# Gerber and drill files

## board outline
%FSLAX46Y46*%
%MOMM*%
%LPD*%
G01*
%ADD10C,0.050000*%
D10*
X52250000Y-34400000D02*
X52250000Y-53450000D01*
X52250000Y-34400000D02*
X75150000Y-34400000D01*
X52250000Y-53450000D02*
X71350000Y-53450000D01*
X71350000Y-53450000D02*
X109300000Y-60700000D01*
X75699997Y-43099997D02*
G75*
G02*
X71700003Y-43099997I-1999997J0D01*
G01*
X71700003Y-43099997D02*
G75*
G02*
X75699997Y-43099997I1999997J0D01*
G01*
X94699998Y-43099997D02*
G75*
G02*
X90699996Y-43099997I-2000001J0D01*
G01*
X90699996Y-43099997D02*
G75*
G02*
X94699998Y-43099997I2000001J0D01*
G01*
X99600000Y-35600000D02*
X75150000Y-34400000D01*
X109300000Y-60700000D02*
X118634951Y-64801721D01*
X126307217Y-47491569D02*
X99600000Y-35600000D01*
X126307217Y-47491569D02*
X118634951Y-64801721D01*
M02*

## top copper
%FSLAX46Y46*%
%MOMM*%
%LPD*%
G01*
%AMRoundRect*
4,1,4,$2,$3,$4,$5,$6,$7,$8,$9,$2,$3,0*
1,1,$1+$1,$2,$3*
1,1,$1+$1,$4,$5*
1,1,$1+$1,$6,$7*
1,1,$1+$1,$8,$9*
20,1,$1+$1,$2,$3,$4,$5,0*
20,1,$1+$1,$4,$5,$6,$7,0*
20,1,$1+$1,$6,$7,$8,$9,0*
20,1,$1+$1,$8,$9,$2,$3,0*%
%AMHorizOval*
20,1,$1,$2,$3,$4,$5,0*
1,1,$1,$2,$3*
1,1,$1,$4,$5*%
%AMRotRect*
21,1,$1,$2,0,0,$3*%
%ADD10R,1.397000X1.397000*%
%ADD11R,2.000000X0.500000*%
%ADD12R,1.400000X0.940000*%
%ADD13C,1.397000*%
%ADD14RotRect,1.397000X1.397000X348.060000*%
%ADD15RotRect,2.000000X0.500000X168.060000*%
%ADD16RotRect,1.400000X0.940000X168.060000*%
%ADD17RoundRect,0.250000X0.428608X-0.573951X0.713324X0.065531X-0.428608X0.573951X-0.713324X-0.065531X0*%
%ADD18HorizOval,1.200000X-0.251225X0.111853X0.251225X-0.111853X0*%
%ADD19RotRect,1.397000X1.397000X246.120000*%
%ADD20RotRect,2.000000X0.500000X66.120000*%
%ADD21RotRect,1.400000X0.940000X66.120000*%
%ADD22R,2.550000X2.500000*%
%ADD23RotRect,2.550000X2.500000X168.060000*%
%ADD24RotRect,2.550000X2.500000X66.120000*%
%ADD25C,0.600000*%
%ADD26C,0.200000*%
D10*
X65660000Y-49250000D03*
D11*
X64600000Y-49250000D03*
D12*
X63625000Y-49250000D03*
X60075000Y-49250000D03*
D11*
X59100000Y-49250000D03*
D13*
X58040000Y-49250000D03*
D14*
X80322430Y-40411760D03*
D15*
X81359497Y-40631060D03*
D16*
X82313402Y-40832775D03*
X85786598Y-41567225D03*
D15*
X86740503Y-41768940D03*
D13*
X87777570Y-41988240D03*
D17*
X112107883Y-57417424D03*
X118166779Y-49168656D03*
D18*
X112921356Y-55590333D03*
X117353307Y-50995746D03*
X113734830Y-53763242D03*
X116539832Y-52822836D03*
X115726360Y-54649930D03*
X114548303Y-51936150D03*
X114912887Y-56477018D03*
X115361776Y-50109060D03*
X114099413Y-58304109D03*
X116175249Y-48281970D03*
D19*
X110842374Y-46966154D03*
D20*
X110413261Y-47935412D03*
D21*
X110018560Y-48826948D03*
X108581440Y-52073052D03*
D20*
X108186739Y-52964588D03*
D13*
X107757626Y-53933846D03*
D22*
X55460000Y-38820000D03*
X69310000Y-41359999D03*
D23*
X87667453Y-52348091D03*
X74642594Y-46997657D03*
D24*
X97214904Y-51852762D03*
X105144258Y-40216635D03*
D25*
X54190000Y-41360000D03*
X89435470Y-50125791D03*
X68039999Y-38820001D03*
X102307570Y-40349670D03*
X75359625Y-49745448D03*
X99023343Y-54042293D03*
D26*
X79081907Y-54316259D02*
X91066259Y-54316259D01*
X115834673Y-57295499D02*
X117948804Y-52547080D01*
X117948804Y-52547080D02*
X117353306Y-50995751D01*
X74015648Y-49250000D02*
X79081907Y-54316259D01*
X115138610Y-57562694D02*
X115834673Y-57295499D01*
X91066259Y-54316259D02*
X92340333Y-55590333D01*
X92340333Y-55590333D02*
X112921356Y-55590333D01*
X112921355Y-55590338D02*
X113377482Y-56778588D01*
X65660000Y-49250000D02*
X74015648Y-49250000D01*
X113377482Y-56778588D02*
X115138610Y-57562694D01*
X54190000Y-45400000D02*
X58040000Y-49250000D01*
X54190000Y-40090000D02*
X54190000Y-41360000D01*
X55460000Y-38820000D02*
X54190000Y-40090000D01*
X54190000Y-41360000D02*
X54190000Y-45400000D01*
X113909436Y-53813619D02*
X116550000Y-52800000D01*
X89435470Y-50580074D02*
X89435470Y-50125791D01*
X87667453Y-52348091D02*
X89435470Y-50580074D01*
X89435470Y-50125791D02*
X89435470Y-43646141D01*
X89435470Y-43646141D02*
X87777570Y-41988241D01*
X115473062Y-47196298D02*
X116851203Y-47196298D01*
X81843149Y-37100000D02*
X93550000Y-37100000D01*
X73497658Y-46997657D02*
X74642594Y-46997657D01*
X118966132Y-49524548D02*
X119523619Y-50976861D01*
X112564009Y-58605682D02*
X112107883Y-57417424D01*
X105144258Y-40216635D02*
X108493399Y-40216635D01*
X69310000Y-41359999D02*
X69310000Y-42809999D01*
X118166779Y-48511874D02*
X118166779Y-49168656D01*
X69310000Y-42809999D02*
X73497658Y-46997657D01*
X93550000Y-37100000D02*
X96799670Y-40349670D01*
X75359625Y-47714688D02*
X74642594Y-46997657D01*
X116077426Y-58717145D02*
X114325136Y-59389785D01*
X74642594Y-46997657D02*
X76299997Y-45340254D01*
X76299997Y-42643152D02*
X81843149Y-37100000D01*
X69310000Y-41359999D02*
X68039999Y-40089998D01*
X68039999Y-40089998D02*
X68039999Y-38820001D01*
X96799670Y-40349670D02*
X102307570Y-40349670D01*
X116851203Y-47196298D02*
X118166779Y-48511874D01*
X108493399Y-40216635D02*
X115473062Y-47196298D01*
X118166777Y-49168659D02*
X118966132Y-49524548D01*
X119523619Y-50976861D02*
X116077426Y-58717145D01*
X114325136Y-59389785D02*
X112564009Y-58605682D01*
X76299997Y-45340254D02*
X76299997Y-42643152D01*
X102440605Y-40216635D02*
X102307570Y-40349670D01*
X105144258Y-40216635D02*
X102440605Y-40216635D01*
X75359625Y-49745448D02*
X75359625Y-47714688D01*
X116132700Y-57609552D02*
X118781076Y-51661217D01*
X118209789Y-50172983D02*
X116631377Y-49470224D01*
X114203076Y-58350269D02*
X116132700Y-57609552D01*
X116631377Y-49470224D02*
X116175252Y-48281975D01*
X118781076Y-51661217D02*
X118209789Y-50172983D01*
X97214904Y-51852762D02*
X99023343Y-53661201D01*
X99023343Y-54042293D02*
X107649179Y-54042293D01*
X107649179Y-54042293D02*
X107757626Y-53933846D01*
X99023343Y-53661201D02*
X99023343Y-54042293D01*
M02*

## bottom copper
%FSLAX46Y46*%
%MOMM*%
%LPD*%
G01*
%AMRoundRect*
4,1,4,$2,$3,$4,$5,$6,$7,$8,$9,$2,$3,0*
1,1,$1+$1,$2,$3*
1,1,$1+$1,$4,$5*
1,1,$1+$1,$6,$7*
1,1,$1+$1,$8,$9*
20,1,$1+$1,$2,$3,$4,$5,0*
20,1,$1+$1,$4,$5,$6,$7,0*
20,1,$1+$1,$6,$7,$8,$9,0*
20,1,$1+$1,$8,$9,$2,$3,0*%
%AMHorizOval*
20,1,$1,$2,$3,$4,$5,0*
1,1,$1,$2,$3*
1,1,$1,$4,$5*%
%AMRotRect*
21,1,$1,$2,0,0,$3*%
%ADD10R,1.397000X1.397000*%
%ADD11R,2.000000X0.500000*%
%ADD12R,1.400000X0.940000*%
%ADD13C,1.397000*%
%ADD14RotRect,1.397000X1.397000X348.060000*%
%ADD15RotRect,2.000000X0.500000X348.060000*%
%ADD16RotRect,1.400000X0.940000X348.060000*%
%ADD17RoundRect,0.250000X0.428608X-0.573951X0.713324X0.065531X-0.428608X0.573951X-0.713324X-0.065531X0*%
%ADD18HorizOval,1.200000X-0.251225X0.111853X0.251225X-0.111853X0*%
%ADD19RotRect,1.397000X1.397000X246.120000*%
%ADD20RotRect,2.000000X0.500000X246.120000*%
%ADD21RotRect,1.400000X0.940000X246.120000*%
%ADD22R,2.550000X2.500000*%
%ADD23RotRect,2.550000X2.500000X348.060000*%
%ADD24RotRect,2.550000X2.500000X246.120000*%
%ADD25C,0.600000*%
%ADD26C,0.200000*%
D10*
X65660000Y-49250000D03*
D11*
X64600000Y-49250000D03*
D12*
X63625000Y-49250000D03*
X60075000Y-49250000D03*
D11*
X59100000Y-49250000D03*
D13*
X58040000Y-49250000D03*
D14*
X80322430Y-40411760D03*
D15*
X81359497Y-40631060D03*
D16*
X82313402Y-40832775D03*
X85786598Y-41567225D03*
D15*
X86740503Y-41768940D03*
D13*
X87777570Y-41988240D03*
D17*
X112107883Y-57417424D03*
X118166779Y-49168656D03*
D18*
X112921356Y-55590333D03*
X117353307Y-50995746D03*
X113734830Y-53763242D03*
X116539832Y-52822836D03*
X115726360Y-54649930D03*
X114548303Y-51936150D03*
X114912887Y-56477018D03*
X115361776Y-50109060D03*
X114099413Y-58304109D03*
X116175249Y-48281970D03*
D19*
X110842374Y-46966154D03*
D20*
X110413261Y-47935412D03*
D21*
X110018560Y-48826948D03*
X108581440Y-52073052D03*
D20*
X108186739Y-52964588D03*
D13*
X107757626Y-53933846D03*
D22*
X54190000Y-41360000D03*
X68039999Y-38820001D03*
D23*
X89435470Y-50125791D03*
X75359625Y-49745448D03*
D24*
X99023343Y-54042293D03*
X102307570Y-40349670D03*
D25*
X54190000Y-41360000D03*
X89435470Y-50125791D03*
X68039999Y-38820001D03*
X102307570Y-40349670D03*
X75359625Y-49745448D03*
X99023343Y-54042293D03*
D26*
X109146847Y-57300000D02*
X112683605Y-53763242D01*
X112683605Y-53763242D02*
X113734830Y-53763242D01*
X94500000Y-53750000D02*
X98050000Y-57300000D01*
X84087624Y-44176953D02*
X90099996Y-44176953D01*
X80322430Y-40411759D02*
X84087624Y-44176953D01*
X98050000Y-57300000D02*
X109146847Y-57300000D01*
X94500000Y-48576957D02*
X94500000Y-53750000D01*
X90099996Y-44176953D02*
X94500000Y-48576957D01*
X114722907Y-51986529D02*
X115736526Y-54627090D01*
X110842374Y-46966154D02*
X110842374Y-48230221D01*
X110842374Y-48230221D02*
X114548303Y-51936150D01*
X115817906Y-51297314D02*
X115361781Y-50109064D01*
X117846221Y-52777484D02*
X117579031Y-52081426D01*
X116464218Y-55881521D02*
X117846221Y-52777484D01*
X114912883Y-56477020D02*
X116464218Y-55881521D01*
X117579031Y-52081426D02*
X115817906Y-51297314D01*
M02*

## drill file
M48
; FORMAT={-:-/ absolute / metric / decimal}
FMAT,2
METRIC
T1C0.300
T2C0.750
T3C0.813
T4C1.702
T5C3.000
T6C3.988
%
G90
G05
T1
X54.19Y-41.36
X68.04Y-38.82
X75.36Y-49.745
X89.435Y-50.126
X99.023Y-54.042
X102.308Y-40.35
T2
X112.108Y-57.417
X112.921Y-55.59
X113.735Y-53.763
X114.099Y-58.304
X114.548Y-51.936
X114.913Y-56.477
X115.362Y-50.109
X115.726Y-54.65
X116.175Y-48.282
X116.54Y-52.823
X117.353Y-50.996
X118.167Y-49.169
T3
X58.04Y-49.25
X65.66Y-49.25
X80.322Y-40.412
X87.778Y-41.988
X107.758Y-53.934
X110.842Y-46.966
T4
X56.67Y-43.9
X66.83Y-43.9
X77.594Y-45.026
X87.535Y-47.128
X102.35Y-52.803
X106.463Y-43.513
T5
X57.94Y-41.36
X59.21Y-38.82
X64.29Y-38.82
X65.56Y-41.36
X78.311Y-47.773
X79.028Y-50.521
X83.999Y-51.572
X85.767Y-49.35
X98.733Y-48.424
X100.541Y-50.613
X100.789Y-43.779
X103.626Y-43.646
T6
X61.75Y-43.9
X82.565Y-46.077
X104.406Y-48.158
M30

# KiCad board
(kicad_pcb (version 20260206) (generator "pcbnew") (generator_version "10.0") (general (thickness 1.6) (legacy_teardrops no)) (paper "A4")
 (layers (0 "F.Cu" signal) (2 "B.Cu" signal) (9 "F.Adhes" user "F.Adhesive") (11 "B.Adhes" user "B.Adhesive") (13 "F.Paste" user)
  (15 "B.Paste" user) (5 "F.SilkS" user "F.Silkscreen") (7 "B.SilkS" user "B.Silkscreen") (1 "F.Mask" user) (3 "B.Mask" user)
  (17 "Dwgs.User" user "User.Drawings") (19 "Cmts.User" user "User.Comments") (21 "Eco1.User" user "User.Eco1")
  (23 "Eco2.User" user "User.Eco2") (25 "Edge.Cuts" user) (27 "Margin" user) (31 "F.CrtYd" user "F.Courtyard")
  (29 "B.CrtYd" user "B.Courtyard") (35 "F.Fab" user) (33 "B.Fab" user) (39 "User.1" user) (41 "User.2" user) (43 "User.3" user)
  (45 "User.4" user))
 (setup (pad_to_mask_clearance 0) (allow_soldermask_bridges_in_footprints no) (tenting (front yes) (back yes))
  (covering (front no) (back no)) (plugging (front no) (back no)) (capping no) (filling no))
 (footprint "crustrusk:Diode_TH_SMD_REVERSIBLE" (layer "F.Cu") (at 61.85 49.25 180)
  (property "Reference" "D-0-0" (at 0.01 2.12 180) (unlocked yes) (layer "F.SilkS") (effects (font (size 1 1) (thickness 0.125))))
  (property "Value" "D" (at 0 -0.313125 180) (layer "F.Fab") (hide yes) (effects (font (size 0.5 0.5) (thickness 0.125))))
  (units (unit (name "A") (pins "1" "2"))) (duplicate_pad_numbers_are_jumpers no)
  (pad "1" thru_hole rect (at -3.81 0 180) (size 1.397 1.397) (drill 0.8128) (layers "*.Cu" "*.Mask") (remove_unused_layers no)
   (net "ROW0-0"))
  (pad "1" smd rect (at -2.75 0) (size 2 0.5) (layers "F.Cu") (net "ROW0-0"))
  (pad "1" smd rect (at -2.75 0 180) (size 2 0.5) (layers "B.Cu") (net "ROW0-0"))
  (pad "1" smd rect (at -1.775 0) (size 1.4 0.94) (layers "F.Cu" "F.Mask" "F.Paste") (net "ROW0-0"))
  (pad "1" smd rect (at -1.775 0 180) (size 1.4 0.94) (layers "B.Cu" "B.Mask" "B.Paste") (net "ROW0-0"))
  (pad "2" smd rect (at 1.775 0) (size 1.4 0.94) (layers "F.Cu" "F.Mask" "F.Paste") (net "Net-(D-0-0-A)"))
  (pad "2" smd rect (at 1.775 0 180) (size 1.4 0.94) (layers "B.Cu" "B.Mask" "B.Paste") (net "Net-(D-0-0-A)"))
  (pad "2" smd rect (at 2.75 0) (size 2 0.5) (layers "F.Cu") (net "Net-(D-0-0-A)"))
  (pad "2" smd rect (at 2.75 0 180) (size 2 0.5) (layers "B.Cu") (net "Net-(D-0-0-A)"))
  (pad "2" thru_hole circle (at 3.81 0 180) (size 1.397 1.397) (drill 0.8128) (layers "*.Cu" "*.Mask") (remove_unused_layers no)
   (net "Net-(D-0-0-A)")))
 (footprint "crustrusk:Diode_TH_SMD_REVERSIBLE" (layer "F.Cu") (at 84.05 41.2 -11.94)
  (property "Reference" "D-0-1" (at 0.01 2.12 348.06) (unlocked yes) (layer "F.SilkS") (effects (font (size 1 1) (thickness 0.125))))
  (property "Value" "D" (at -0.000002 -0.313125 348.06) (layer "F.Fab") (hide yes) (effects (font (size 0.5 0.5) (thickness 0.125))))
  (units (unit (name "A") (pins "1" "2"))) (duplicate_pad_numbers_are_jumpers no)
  (pad "1" thru_hole rect (at -3.81 0 348.06) (size 1.397 1.397) (drill 0.8128) (layers "*.Cu" "*.Mask") (remove_unused_layers no)
   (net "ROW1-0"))
  (pad "1" smd rect (at -2.75 0 168.06) (size 2 0.5) (layers "F.Cu") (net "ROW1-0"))
  (pad "1" smd rect (at -2.75 0 348.06) (size 2 0.5) (layers "B.Cu") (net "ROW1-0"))
  (pad "1" smd rect (at -1.775001 0 168.06) (size 1.4 0.94) (layers "F.Cu" "F.Mask" "F.Paste") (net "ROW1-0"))
  (pad "1" smd rect (at -1.775001 0 348.06) (size 1.4 0.94) (layers "B.Cu" "B.Mask" "B.Paste") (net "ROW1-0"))
  (pad "2" smd rect (at 1.775001 0 168.06) (size 1.4 0.94) (layers "F.Cu" "F.Mask" "F.Paste") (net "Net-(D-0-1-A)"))
  (pad "2" smd rect (at 1.775001 0 348.06) (size 1.4 0.94) (layers "B.Cu" "B.Mask" "B.Paste") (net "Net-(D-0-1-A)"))
  (pad "2" smd rect (at 2.75 0 168.06) (size 2 0.5) (layers "F.Cu") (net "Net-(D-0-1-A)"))
  (pad "2" smd rect (at 2.75 0 348.06) (size 2 0.5) (layers "B.Cu") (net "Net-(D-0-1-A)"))
  (pad "2" thru_hole circle (at 3.81 0 348.06) (size 1.397 1.397) (drill 0.8128) (layers "*.Cu" "*.Mask") (remove_unused_layers no)
   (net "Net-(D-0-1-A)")))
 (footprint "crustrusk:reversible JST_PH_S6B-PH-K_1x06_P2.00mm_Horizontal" (layer "F.Cu") (at 112.107883 57.417424 66)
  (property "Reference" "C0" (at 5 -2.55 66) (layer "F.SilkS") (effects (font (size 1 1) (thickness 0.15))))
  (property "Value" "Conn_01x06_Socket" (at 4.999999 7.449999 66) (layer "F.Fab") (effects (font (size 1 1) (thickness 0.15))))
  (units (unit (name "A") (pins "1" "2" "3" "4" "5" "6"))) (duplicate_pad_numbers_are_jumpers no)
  (pad "1" thru_hole roundrect (at 0 0 66) (size 1.2 1.75) (drill 0.75) (layers "*.Cu" "*.Mask") (remove_unused_layers no)
   (roundrect_rratio 0.208333) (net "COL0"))
  (pad "1" thru_hole roundrect (at 10 2.180001 66) (size 1.2 1.75) (drill 0.75) (layers "*.Cu" "*.Mask") (remove_unused_layers no)
   (roundrect_rratio 0.208333) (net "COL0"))
  (pad "2" thru_hole oval (at 2 0 66) (size 1.2 1.75) (drill 0.75) (layers "*.Cu" "*.Mask") (remove_unused_layers no) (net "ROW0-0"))
  (pad "2" thru_hole oval (at 8.000001 2.180002 66) (size 1.2 1.75) (drill 0.75) (layers "*.Cu" "*.Mask") (remove_unused_layers no)
   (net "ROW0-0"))
  (pad "3" thru_hole oval (at 4 0 66) (size 1.2 1.75) (drill 0.75) (layers "*.Cu" "*.Mask") (remove_unused_layers no) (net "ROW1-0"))
  (pad "3" thru_hole oval (at 6.000001 2.18 66) (size 1.2 1.75) (drill 0.75) (layers "*.Cu" "*.Mask") (remove_unused_layers no)
   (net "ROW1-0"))
  (pad "4" thru_hole oval (at 3.999999 2.180002 66) (size 1.2 1.75) (drill 0.75) (layers "*.Cu" "*.Mask") (remove_unused_layers no)
   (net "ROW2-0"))
  (pad "4" thru_hole oval (at 6.000001 0 66) (size 1.2 1.75) (drill 0.75) (layers "*.Cu" "*.Mask") (remove_unused_layers no) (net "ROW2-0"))
  (pad "5" thru_hole oval (at 2.000002 2.180001 66) (size 1.2 1.75) (drill 0.75) (layers "*.Cu" "*.Mask") (remove_unused_layers no)
   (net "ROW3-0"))
  (pad "5" thru_hole oval (at 8 0 66) (size 1.2 1.75) (drill 0.75) (layers "*.Cu" "*.Mask") (remove_unused_layers no) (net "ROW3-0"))
  (pad "6" thru_hole oval (at 0.000001 2.18 66) (size 1.2 1.75) (drill 0.75) (layers "*.Cu" "*.Mask") (remove_unused_layers no)
   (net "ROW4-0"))
  (pad "6" thru_hole oval (at 9.999999 0 66) (size 1.2 1.75) (drill 0.75) (layers "*.Cu" "*.Mask") (remove_unused_layers no) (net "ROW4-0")))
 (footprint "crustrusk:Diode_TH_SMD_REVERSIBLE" (layer "F.Cu") (at 109.3 50.45 -113.88)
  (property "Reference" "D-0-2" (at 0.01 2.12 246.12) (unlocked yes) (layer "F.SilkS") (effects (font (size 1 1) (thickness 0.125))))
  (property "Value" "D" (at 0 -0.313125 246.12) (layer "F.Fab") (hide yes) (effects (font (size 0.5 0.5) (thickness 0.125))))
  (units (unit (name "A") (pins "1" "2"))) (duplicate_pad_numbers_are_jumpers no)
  (pad "1" thru_hole rect (at -3.81 -0.000001 246.12) (size 1.397 1.397) (drill 0.8128) (layers "*.Cu" "*.Mask") (remove_unused_layers no)
   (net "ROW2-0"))
  (pad "1" smd rect (at -2.75 0.000001 66.12) (size 2 0.5) (layers "F.Cu") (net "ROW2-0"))
  (pad "1" smd rect (at -2.75 0.000001 246.12) (size 2 0.5) (layers "B.Cu") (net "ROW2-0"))
  (pad "1" smd rect (at -1.775 0 66.12) (size 1.4 0.94) (layers "F.Cu" "F.Mask" "F.Paste") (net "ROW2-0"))
  (pad "1" smd rect (at -1.775 0 246.12) (size 1.4 0.94) (layers "B.Cu" "B.Mask" "B.Paste") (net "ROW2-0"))
  (pad "2" smd rect (at 1.775 0 66.12) (size 1.4 0.94) (layers "F.Cu" "F.Mask" "F.Paste") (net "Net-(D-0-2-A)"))
  (pad "2" smd rect (at 1.775 0 246.12) (size 1.4 0.94) (layers "B.Cu" "B.Mask" "B.Paste") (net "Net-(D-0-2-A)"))
  (pad "2" smd rect (at 2.75 -0.000001 66.12) (size 2 0.5) (layers "F.Cu") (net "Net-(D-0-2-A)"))
  (pad "2" smd rect (at 2.75 -0.000001 246.12) (size 2 0.5) (layers "B.Cu") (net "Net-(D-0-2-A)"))
  (pad "2" thru_hole circle (at 3.81 0.000001 246.12) (size 1.397 1.397) (drill 0.8128) (layers "*.Cu" "*.Mask") (remove_unused_layers no)
   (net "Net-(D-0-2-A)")))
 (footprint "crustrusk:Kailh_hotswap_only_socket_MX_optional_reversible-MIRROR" (layer "B.Cu") (at 61.75 43.9 180)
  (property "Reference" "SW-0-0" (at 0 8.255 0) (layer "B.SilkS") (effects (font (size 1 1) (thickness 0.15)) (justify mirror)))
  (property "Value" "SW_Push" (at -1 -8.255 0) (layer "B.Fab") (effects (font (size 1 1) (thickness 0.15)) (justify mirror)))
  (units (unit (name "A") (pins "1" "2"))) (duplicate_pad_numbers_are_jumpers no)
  (pad "" np_thru_hole circle (at -5.08 0 180) (size 1.7018 1.7018) (drill 1.7018) (layers "*.Cu" "*.Mask"))
  (pad "" np_thru_hole circle (at -3.81 2.54) (size 3 3) (drill 3) (layers "*.Cu" "*.Mask"))
  (pad "" np_thru_hole circle (at -2.54 5.079998 180) (size 3 3) (drill 3) (layers "*.Cu" "*.Mask"))
  (pad "" np_thru_hole circle (at 0 0 180) (size 3.9878 3.9878) (drill 3.9878) (layers "*.Cu" "*.Mask"))
  (pad "" np_thru_hole circle (at 2.540002 5.080001) (size 3 3) (drill 3) (layers "*.Cu" "*.Mask"))
  (pad "" np_thru_hole circle (at 3.81 2.54 180) (size 3 3) (drill 3) (layers "*.Cu" "*.Mask"))
  (pad "" np_thru_hole circle (at 5.08 0 180) (size 1.7018 1.7018) (drill 1.7018) (layers "*.Cu" "*.Mask"))
  (pad "1" smd rect (at 6.29 5.08) (size 2.55 2.5) (layers "F.Cu" "F.Mask" "F.Paste") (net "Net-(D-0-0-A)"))
  (pad "1" smd rect (at 7.56 2.54 180) (size 2.55 2.5) (layers "B.Cu" "B.Mask" "B.Paste") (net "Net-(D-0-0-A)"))
  (pad "2" smd rect (at -7.56 2.540001) (size 2.55 2.5) (layers "F.Cu" "F.Mask" "F.Paste") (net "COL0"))
  (pad "2" smd rect (at -6.289999 5.079999 180) (size 2.55 2.5) (layers "B.Cu" "B.Mask" "B.Paste") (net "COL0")))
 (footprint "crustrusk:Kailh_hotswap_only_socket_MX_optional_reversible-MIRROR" (layer "B.Cu") (at 82.564526 46.076677 -11.94)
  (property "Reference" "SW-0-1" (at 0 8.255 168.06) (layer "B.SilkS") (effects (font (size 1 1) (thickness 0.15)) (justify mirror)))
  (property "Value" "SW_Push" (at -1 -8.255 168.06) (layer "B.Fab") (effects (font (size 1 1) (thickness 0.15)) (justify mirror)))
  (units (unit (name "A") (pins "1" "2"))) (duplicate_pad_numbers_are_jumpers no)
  (pad "" np_thru_hole circle (at -5.079999 0 348.06) (size 1.7018 1.7018) (drill 1.7018) (layers "*.Cu" "*.Mask"))
  (pad "" np_thru_hole circle (at -3.81 2.54 168.06) (size 3 3) (drill 3) (layers "*.Cu" "*.Mask"))
  (pad "" np_thru_hole circle (at -2.54 5.079997 348.06) (size 3 3) (drill 3) (layers "*.Cu" "*.Mask"))
  (pad "" np_thru_hole circle (at 0 0 348.06) (size 3.9878 3.9878) (drill 3.9878) (layers "*.Cu" "*.Mask"))
  (pad "" np_thru_hole circle (at 2.540002 5.080001 168.06) (size 3 3) (drill 3) (layers "*.Cu" "*.Mask"))
  (pad "" np_thru_hole circle (at 3.81 2.54 348.06) (size 3 3) (drill 3) (layers "*.Cu" "*.Mask"))
  (pad "" np_thru_hole circle (at 5.079999 0 348.06) (size 1.7018 1.7018) (drill 1.7018) (layers "*.Cu" "*.Mask"))
  (pad "1" smd rect (at 6.29 5.08 168.06) (size 2.55 2.5) (layers "F.Cu" "F.Mask" "F.Paste") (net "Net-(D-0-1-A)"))
  (pad "1" smd rect (at 7.56 2.54 348.06) (size 2.55 2.5) (layers "B.Cu" "B.Mask" "B.Paste") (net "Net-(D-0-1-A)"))
  (pad "2" smd rect (at -7.56 2.540001 168.06) (size 2.55 2.5) (layers "F.Cu" "F.Mask" "F.Paste") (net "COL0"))
  (pad "2" smd rect (at -6.289999 5.079999 348.06) (size 2.55 2.5) (layers "B.Cu" "B.Mask" "B.Paste") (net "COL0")))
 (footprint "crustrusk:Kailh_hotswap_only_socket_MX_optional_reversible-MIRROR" (layer "B.Cu") (at 104.406365 48.157713 -113.88)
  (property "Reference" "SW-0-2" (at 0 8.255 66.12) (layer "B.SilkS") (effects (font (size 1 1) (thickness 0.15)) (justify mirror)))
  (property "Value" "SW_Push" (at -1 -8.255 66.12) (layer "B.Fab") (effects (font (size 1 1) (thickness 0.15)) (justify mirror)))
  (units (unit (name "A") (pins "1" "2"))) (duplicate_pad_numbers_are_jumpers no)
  (pad "" np_thru_hole circle (at -5.08 0 246.12) (size 1.7018 1.7018) (drill 1.7018) (layers "*.Cu" "*.Mask"))
  (pad "" np_thru_hole circle (at -3.81 2.54 66.12) (size 3 3) (drill 3) (layers "*.Cu" "*.Mask"))
  (pad "" np_thru_hole circle (at -2.54 5.079998 246.12) (size 3 3) (drill 3) (layers "*.Cu" "*.Mask"))
  (pad "" np_thru_hole circle (at 0 0 246.12) (size 3.9878 3.9878) (drill 3.9878) (layers "*.Cu" "*.Mask"))
  (pad "" np_thru_hole circle (at 2.540002 5.080001 66.12) (size 3 3) (drill 3) (layers "*.Cu" "*.Mask"))
  (pad "" np_thru_hole circle (at 3.81 2.54 246.12) (size 3 3) (drill 3) (layers "*.Cu" "*.Mask"))
  (pad "" np_thru_hole circle (at 5.08 0 246.12) (size 1.7018 1.7018) (drill 1.7018) (layers "*.Cu" "*.Mask"))
  (pad "1" smd rect (at 6.29 5.08 66.12) (size 2.55 2.5) (layers "F.Cu" "F.Mask" "F.Paste") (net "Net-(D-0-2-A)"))
  (pad "1" smd rect (at 7.56 2.54 246.12) (size 2.55 2.5) (layers "B.Cu" "B.Mask" "B.Paste") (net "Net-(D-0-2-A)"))
  (pad "2" smd rect (at -7.56 2.540001 66.12) (size 2.55 2.5) (layers "F.Cu" "F.Mask" "F.Paste") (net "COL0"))
  (pad "2" smd rect (at -6.289999 5.079999 246.12) (size 2.55 2.5) (layers "B.Cu" "B.Mask" "B.Paste") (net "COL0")))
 (gr_line (start 52.25 34.4) (end 52.25 53.45) (stroke (width 0.05) (type default)) (layer "Edge.Cuts"))
 (gr_line (start 52.25 34.4) (end 75.15 34.4) (stroke (width 0.05) (type default)) (layer "Edge.Cuts"))
 (gr_line (start 52.25 53.45) (end 71.35 53.45) (stroke (width 0.05) (type default)) (layer "Edge.Cuts"))
 (gr_line (start 71.35 53.45) (end 109.3 60.7) (stroke (width 0.05) (type default)) (layer "Edge.Cuts"))
 (gr_circle (center 73.7 43.099997) (end 75.699997 43.099997) (stroke (width 0.05) (type default)) (fill no) (layer "Edge.Cuts"))
 (gr_circle (center 92.699997 43.099997) (end 94.699998 43.099997) (stroke (width 0.05) (type default)) (fill no) (layer "Edge.Cuts"))
 (gr_line (start 99.6 35.6) (end 75.15 34.4) (stroke (width 0.05) (type default)) (layer "Edge.Cuts"))
 (gr_line (start 109.3 60.7) (end 118.634951 64.801721) (stroke (width 0.05) (type default)) (layer "Edge.Cuts"))
 (gr_line (start 126.307217 47.491569) (end 99.6 35.6) (stroke (width 0.05) (type default)) (layer "Edge.Cuts"))
 (gr_line (start 126.307217 47.491569) (end 118.634951 64.801721) (stroke (width 0.05) (type default)) (layer "Edge.Cuts"))
 (segment (start 79.081907 54.316259) (end 91.066259 54.316259) (width 0.2) (layer "F.Cu") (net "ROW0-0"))
 (segment (start 115.834673 57.295499) (end 117.948804 52.54708) (width 0.2) (layer "F.Cu") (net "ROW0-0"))
 (segment (start 117.948804 52.54708) (end 117.353306 50.995751) (width 0.2) (layer "F.Cu") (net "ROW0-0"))
 (segment (start 74.015648 49.25) (end 79.081907 54.316259) (width 0.2) (layer "F.Cu") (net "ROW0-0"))
 (segment (start 115.13861 57.562694) (end 115.834673 57.295499) (width 0.2) (layer "F.Cu") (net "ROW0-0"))
 (segment (start 91.066259 54.316259) (end 92.340333 55.590333) (width 0.2) (layer "F.Cu") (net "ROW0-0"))
 (segment (start 92.340333 55.590333) (end 112.921356 55.590333) (width 0.2) (layer "F.Cu") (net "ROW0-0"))
 (segment (start 112.921355 55.590338) (end 113.377482 56.778588) (width 0.2) (layer "F.Cu") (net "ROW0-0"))
 (segment (start 65.66 49.25) (end 74.015648 49.25) (width 0.2) (layer "F.Cu") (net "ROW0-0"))
 (segment (start 113.377482 56.778588) (end 115.13861 57.562694) (width 0.2) (layer "F.Cu") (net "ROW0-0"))
 (segment (start 54.19 45.4) (end 58.04 49.25) (width 0.2) (layer "F.Cu") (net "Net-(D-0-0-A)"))
 (segment (start 54.19 40.09) (end 54.19 41.36) (width 0.2) (layer "F.Cu") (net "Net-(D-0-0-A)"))
 (segment (start 55.46 38.82) (end 54.19 40.09) (width 0.2) (layer "F.Cu") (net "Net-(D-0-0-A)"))
 (segment (start 54.19 41.36) (end 54.19 45.4) (width 0.2) (layer "F.Cu") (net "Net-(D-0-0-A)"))
 (via (at 54.19 41.36) (size 0.6) (drill 0.3) (layers "F.Cu" "B.Cu") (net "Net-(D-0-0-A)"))
 (segment (start 113.909436 53.813619) (end 116.55 52.8) (width 0.2) (layer "F.Cu") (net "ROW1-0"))
 (segment (start 109.146847 57.3) (end 112.683605 53.763242) (width 0.2) (layer "B.Cu") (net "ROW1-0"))
 (segment (start 112.683605 53.763242) (end 113.73483 53.763242) (width 0.2) (layer "B.Cu") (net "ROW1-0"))
 (segment (start 94.5 53.75) (end 98.05 57.3) (width 0.2) (layer "B.Cu") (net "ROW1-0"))
 (segment (start 84.087624 44.176953) (end 90.099996 44.176953) (width 0.2) (layer "B.Cu") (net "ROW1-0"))
 (segment (start 80.32243 40.411759) (end 84.087624 44.176953) (width 0.2) (layer "B.Cu") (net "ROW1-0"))
 (segment (start 98.05 57.3) (end 109.146847 57.3) (width 0.2) (layer "B.Cu") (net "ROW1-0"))
 (segment (start 94.5 48.576957) (end 94.5 53.75) (width 0.2) (layer "B.Cu") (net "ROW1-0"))
 (segment (start 90.099996 44.176953) (end 94.5 48.576957) (width 0.2) (layer "B.Cu") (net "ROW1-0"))
 (segment (start 89.43547 50.580074) (end 89.43547 50.125791) (width 0.2) (layer "F.Cu") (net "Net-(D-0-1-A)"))
 (segment (start 87.667453 52.348091) (end 89.43547 50.580074) (width 0.2) (layer "F.Cu") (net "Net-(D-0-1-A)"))
 (segment (start 89.43547 50.125791) (end 89.43547 43.646141) (width 0.2) (layer "F.Cu") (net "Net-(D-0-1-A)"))
 (segment (start 89.43547 43.646141) (end 87.77757 41.988241) (width 0.2) (layer "F.Cu") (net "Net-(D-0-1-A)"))
 (via (at 89.43547 50.125791) (size 0.6) (drill 0.3) (layers "F.Cu" "B.Cu") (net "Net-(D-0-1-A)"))
 (segment (start 115.473062 47.196298) (end 116.851203 47.196298) (width 0.2) (layer "F.Cu") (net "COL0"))
 (segment (start 81.843149 37.1) (end 93.55 37.1) (width 0.2) (layer "F.Cu") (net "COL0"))
 (segment (start 73.497658 46.997657) (end 74.642594 46.997657) (width 0.2) (layer "F.Cu") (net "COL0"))
 (segment (start 118.966132 49.524548) (end 119.523619 50.976861) (width 0.2) (layer "F.Cu") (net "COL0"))
 (segment (start 112.564009 58.605682) (end 112.107883 57.417424) (width 0.2) (layer "F.Cu") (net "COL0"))
 (segment (start 105.144258 40.216635) (end 108.493399 40.216635) (width 0.2) (layer "F.Cu") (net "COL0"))
 (segment (start 69.31 41.359999) (end 69.31 42.809999) (width 0.2) (layer "F.Cu") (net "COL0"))
 (segment (start 118.166779 48.511874) (end 118.166779 49.168656) (width 0.2) (layer "F.Cu") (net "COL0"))
 (segment (start 69.31 42.809999) (end 73.497658 46.997657) (width 0.2) (layer "F.Cu") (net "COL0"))
 (segment (start 93.55 37.1) (end 96.79967 40.34967) (width 0.2) (layer "F.Cu") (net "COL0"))
 (segment (start 75.359625 47.714688) (end 74.642594 46.997657) (width 0.2) (layer "F.Cu") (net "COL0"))
 (segment (start 116.077426 58.717145) (end 114.325136 59.389785) (width 0.2) (layer "F.Cu") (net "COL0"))
 (segment (start 74.642594 46.997657) (end 76.299997 45.340254) (width 0.2) (layer "F.Cu") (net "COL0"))
 (segment (start 76.299997 42.643152) (end 81.843149 37.1) (width 0.2) (layer "F.Cu") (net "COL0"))
 (segment (start 69.31 41.359999) (end 68.039999 40.089998) (width 0.2) (layer "F.Cu") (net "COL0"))
 (segment (start 68.039999 40.089998) (end 68.039999 38.820001) (width 0.2) (layer "F.Cu") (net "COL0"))
 (segment (start 96.79967 40.34967) (end 102.30757 40.34967) (width 0.2) (layer "F.Cu") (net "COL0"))
 (segment (start 116.851203 47.196298) (end 118.166779 48.511874) (width 0.2) (layer "F.Cu") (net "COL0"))
 (segment (start 108.493399 40.216635) (end 115.473062 47.196298) (width 0.2) (layer "F.Cu") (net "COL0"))
 (segment (start 118.166777 49.168659) (end 118.966132 49.524548) (width 0.2) (layer "F.Cu") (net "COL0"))
 (segment (start 119.523619 50.976861) (end 116.077426 58.717145) (width 0.2) (layer "F.Cu") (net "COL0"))
 (segment (start 114.325136 59.389785) (end 112.564009 58.605682) (width 0.2) (layer "F.Cu") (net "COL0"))
 (segment (start 76.299997 45.340254) (end 76.299997 42.643152) (width 0.2) (layer "F.Cu") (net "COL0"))
 (segment (start 102.440605 40.216635) (end 102.30757 40.34967) (width 0.2) (layer "F.Cu") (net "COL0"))
 (segment (start 105.144258 40.216635) (end 102.440605 40.216635) (width 0.2) (layer "F.Cu") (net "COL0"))
 (segment (start 75.359625 49.745448) (end 75.359625 47.714688) (width 0.2) (layer "F.Cu") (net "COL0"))
 (via (at 68.039999 38.820001) (size 0.6) (drill 0.3) (layers "F.Cu" "B.Cu") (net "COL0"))
 (via (at 102.30757 40.34967) (size 0.6) (drill 0.3) (layers "F.Cu" "B.Cu") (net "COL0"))
 (via (at 75.359625 49.745448) (size 0.6) (drill 0.3) (layers "F.Cu" "B.Cu") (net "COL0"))
 (segment (start 114.722907 51.986529) (end 115.736526 54.62709) (width 0.2) (layer "B.Cu") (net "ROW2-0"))
 (segment (start 110.842374 46.966154) (end 110.842374 48.230221) (width 0.2) (layer "B.Cu") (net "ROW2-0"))
 (segment (start 110.842374 48.230221) (end 114.548303 51.93615) (width 0.2) (layer "B.Cu") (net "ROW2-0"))
 (segment (start 115.817906 51.297314) (end 115.361781 50.109064) (width 0.2) (layer "B.Cu") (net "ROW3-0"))
 (segment (start 117.846221 52.777484) (end 117.579031 52.081426) (width 0.2) (layer "B.Cu") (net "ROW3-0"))
 (segment (start 116.464218 55.881521) (end 117.846221 52.777484) (width 0.2) (layer "B.Cu") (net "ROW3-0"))
 (segment (start 114.912883 56.47702) (end 116.464218 55.881521) (width 0.2) (layer "B.Cu") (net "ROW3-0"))
 (segment (start 117.579031 52.081426) (end 115.817906 51.297314) (width 0.2) (layer "B.Cu") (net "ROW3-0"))
 (segment (start 116.1327 57.609552) (end 118.781076 51.661217) (width 0.2) (layer "F.Cu") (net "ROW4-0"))
 (segment (start 118.209789 50.172983) (end 116.631377 49.470224) (width 0.2) (layer "F.Cu") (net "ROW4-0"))
 (segment (start 114.203076 58.350269) (end 116.1327 57.609552) (width 0.2) (layer "F.Cu") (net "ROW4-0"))
 (segment (start 116.631377 49.470224) (end 116.175252 48.281975) (width 0.2) (layer "F.Cu") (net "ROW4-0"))
 (segment (start 118.781076 51.661217) (end 118.209789 50.172983) (width 0.2) (layer "F.Cu") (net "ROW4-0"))
 (segment (start 97.214904 51.852762) (end 99.023343 53.661201) (width 0.2) (layer "F.Cu") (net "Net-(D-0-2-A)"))
 (segment (start 99.023343 54.042293) (end 107.649179 54.042293) (width 0.2) (layer "F.Cu") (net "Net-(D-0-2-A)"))
 (segment (start 107.649179 54.042293) (end 107.757626 53.933846) (width 0.2) (layer "F.Cu") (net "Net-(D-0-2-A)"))
 (segment (start 99.023343 53.661201) (end 99.023343 54.042293) (width 0.2) (layer "F.Cu") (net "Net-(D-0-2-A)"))
 (via (at 99.023343 54.042293) (size 0.6) (drill 0.3) (layers "F.Cu" "B.Cu") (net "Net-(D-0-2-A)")))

